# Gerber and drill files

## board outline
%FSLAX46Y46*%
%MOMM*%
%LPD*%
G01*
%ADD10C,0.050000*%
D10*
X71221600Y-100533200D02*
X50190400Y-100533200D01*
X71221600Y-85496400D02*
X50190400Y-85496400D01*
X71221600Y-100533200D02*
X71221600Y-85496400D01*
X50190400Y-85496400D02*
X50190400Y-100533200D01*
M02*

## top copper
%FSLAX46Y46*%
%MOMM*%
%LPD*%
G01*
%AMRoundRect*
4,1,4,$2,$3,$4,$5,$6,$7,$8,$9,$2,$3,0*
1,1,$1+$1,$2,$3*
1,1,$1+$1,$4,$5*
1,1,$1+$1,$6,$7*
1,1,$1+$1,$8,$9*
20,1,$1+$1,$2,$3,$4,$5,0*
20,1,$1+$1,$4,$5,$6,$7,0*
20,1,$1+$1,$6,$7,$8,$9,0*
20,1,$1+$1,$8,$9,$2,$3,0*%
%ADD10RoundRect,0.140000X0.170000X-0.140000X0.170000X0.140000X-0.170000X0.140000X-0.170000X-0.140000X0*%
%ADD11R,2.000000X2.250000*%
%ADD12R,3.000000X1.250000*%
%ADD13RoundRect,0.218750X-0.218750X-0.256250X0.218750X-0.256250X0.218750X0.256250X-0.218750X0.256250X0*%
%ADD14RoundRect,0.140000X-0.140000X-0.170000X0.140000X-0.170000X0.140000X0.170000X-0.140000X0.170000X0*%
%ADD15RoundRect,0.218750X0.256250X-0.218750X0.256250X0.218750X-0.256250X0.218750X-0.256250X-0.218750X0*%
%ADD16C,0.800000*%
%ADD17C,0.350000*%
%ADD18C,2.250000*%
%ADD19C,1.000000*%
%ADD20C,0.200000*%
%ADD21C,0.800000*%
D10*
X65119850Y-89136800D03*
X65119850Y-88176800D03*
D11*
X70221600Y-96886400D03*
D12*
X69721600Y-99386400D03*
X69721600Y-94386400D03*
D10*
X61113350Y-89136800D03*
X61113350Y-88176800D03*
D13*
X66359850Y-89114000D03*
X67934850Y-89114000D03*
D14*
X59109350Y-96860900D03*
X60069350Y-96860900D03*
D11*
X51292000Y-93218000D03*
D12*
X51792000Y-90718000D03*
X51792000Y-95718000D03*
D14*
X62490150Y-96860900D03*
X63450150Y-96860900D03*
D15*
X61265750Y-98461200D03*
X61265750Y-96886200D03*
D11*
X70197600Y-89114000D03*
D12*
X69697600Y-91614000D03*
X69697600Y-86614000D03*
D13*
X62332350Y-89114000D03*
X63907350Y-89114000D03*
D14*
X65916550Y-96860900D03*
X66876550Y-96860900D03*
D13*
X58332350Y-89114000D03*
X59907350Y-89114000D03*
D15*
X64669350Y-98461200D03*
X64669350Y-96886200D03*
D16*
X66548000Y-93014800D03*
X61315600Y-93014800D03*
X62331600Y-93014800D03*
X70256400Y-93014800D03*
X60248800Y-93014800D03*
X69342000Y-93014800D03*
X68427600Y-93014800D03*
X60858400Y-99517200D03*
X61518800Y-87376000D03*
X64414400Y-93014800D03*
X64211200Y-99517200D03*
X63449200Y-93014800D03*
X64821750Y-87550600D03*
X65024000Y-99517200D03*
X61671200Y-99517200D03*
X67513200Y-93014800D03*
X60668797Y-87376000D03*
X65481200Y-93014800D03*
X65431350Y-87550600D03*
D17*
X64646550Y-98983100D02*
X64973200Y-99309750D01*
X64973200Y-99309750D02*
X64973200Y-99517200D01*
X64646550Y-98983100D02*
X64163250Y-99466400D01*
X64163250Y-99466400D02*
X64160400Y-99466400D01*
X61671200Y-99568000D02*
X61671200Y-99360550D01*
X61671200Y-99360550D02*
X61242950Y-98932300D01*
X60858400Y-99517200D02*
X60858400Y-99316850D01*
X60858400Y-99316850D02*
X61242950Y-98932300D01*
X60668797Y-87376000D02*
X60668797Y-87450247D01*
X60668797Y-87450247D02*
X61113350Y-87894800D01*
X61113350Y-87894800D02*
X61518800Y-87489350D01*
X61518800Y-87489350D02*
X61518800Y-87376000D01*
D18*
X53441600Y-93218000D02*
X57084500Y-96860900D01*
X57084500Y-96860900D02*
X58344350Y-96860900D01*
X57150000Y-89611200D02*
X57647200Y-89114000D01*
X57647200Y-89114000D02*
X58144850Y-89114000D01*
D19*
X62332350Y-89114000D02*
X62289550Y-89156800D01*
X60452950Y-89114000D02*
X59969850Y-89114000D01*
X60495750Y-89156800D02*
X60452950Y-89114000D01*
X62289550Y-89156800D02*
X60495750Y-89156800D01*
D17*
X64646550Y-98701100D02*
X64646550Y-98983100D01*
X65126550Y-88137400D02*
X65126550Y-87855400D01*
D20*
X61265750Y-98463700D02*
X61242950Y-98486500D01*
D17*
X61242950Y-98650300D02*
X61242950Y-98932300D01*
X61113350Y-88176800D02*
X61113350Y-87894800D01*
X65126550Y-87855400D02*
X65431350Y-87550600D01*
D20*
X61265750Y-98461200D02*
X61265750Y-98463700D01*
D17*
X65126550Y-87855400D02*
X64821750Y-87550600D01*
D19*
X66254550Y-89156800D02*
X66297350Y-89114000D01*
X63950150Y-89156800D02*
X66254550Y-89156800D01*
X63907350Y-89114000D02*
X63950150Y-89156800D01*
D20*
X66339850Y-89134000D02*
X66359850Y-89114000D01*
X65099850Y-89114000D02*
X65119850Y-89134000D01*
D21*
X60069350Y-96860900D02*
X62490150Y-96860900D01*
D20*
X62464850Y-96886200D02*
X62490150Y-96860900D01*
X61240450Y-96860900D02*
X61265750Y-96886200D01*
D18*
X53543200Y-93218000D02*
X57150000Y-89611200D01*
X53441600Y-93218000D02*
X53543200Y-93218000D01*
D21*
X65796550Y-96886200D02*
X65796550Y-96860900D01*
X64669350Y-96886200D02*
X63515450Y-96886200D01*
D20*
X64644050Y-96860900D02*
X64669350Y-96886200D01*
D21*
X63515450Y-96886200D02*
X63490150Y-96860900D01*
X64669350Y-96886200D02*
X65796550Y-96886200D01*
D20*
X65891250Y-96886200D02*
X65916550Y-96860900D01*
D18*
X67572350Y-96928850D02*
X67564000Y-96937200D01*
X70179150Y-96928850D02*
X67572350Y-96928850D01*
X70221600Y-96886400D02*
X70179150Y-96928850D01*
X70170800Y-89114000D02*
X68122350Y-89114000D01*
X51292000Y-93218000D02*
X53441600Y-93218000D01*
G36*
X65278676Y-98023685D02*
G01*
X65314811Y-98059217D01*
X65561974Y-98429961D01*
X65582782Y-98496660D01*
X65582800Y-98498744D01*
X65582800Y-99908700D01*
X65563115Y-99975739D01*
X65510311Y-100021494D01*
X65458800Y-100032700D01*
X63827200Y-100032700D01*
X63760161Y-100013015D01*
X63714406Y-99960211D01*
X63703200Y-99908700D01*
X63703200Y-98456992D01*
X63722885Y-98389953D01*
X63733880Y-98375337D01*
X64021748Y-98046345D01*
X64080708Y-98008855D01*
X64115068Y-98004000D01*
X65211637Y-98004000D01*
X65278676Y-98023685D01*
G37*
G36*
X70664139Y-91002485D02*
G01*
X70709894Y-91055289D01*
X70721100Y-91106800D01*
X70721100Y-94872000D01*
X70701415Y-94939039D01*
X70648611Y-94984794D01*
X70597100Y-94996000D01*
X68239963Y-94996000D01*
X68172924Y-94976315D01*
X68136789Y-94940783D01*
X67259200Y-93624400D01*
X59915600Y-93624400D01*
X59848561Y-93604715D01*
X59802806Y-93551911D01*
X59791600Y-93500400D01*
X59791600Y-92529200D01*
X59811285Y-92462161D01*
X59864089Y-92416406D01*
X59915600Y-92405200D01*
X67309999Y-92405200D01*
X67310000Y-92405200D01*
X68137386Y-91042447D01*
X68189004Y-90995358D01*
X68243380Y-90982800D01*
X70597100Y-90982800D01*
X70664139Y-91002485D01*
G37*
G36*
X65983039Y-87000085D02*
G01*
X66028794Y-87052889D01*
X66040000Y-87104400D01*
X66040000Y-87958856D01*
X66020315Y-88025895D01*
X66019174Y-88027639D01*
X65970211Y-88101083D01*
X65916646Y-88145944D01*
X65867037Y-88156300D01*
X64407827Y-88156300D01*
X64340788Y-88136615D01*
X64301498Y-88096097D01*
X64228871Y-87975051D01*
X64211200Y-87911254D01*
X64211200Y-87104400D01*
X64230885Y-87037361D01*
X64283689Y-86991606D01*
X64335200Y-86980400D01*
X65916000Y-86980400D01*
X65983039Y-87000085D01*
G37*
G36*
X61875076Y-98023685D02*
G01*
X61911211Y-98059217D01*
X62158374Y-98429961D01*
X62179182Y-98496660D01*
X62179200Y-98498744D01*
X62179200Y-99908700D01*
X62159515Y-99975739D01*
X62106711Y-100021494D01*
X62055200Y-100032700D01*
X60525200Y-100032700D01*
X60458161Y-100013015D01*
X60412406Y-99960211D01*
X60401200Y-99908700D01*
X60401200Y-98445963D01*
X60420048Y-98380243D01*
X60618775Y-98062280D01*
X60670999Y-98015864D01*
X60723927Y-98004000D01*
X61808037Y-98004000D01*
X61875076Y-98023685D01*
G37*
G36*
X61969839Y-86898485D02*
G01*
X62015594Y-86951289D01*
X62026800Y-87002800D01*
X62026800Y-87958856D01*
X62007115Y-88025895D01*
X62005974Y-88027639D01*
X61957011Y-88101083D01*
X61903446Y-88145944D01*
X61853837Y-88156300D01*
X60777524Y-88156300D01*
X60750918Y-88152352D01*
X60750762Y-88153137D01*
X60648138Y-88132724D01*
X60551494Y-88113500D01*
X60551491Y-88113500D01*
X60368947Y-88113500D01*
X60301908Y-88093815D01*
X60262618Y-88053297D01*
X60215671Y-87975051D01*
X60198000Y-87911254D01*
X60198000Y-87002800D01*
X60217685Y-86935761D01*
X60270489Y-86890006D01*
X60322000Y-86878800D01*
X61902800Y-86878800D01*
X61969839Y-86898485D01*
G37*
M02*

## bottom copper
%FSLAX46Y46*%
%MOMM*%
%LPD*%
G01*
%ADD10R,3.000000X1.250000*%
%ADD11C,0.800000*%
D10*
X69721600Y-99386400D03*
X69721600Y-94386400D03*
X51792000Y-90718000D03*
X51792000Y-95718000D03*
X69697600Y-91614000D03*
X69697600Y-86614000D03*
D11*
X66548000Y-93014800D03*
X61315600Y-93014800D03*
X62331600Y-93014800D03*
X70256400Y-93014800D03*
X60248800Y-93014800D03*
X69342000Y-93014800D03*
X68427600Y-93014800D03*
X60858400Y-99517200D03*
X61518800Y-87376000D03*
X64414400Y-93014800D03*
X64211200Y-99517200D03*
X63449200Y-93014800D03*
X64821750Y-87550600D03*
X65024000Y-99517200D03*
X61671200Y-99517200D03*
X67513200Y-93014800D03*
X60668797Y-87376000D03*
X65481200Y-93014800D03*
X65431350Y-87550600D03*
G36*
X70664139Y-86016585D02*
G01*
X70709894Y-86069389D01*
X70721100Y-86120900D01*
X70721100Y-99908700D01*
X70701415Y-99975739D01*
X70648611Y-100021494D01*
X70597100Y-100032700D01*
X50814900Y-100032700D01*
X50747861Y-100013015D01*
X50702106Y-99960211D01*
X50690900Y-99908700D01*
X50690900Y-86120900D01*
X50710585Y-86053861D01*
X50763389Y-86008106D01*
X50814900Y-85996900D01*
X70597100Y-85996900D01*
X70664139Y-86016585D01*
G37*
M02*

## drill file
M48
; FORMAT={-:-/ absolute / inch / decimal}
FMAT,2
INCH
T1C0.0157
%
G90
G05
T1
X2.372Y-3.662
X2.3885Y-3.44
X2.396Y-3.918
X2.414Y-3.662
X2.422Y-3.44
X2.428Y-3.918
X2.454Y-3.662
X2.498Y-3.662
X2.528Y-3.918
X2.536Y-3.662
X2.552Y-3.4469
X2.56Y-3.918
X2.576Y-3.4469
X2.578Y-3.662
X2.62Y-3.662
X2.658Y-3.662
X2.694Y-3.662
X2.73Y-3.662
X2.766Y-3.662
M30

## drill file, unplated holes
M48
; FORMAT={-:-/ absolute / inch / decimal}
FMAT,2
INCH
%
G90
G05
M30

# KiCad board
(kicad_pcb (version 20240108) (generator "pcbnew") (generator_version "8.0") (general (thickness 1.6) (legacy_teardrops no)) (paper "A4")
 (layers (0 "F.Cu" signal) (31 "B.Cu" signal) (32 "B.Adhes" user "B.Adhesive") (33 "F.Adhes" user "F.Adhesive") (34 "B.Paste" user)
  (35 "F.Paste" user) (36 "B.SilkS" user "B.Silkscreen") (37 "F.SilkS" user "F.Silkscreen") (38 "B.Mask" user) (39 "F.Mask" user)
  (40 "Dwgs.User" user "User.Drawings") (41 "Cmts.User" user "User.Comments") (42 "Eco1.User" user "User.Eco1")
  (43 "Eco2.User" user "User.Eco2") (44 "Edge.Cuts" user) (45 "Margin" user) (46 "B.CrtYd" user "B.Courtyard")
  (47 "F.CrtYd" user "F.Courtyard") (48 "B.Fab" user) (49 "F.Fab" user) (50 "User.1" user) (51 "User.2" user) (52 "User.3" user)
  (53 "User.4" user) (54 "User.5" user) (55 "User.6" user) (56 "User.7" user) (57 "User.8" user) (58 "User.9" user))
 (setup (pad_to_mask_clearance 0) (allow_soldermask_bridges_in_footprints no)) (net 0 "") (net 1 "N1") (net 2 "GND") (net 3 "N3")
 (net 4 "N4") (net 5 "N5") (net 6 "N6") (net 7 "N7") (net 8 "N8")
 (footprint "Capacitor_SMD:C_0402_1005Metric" (layer "F.Cu") (at 65.11985 88.6568 90)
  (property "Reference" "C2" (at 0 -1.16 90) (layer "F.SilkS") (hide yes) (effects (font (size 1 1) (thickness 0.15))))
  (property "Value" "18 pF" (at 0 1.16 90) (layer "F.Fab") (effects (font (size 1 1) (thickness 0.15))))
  (pad "1" smd roundrect (at -0.48 0 90) (size 0.56 0.62) (layers "F.Cu" "F.Paste" "F.Mask") (roundrect_rratio 0.25) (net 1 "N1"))
  (pad "2" smd roundrect (at 0.48 0 90) (size 0.56 0.62) (layers "F.Cu" "F.Paste" "F.Mask") (roundrect_rratio 0.25) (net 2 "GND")))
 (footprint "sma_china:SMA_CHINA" (layer "F.Cu") (at 71.2216 96.8864 90)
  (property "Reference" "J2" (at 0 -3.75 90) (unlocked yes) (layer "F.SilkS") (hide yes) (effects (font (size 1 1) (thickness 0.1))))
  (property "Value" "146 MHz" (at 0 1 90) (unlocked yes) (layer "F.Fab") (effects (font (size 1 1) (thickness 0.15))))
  (pad "1" smd rect (at 0 -1 90) (size 2.25 2) (layers "F.Cu" "F.Paste" "F.Mask") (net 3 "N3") (thermal_bridge_angle 45))
  (pad "2" smd rect (at -2.5 -1.5 90) (size 1.25 3) (layers "F.Cu" "F.Paste" "F.Mask") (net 2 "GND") (thermal_bridge_angle 45))
  (pad "2" smd rect (at -2.5 -1.5 90) (size 1.25 3) (layers "B.Cu" "F.Paste" "F.Mask") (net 2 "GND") (thermal_bridge_angle 45))
  (pad "2" smd rect (at 2.5 -1.5 90) (size 1.25 3) (layers "F.Cu" "F.Paste" "F.Mask") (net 2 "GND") (thermal_bridge_angle 45))
  (pad "2" smd rect (at 2.5 -1.5 90) (size 1.25 3) (layers "B.Cu" "F.Paste" "F.Mask") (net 2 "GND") (thermal_bridge_angle 45)))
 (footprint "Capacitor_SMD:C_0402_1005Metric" (layer "F.Cu") (at 61.11335 88.6568 90)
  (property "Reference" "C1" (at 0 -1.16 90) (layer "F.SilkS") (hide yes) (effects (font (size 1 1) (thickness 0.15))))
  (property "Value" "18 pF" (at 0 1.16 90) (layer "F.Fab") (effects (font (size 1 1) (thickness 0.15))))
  (pad "1" smd roundrect (at -0.48 0 90) (size 0.56 0.62) (layers "F.Cu" "F.Paste" "F.Mask") (roundrect_rratio 0.25) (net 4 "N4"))
  (pad "2" smd roundrect (at 0.48 0 90) (size 0.56 0.62) (layers "F.Cu" "F.Paste" "F.Mask") (roundrect_rratio 0.25) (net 2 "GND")))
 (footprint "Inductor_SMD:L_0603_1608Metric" (layer "F.Cu") (at 67.14735 89.114)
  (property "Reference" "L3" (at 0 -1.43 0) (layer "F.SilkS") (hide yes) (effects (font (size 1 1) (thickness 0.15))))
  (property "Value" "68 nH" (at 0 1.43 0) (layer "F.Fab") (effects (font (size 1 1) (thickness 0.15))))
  (pad "1" smd roundrect (at -0.7875 0) (size 0.875 0.95) (layers "F.Cu" "F.Paste" "F.Mask") (roundrect_rratio 0.25) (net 1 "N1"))
  (pad "2" smd roundrect (at 0.7875 0) (size 0.875 0.95) (layers "F.Cu" "F.Paste" "F.Mask") (roundrect_rratio 0.25) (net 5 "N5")))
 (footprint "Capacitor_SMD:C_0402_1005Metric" (layer "F.Cu") (at 59.58935 96.8609)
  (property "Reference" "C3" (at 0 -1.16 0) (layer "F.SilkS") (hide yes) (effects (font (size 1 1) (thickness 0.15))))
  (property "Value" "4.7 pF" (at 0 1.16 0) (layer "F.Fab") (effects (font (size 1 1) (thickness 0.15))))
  (pad "1" smd roundrect (at -0.48 0) (size 0.56 0.62) (layers "F.Cu" "F.Paste" "F.Mask") (roundrect_rratio 0.25) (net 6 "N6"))
  (pad "2" smd roundrect (at 0.48 0) (size 0.56 0.62) (layers "F.Cu" "F.Paste" "F.Mask") (roundrect_rratio 0.25) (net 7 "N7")))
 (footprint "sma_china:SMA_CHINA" (layer "F.Cu") (at 50.292 93.218 -90)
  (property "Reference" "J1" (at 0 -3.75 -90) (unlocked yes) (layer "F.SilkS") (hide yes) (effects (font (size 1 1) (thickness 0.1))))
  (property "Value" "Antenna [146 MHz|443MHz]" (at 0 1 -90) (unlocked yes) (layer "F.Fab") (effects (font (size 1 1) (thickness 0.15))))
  (pad "1" smd rect (at 0 -1 270) (size 2.25 2) (layers "F.Cu" "F.Paste" "F.Mask") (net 6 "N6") (thermal_bridge_angle 45))
  (pad "2" smd rect (at -2.5 -1.5 270) (size 1.25 3) (layers "F.Cu" "F.Paste" "F.Mask") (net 2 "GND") (thermal_bridge_angle 45))
  (pad "2" smd rect (at -2.5 -1.5 270) (size 1.25 3) (layers "B.Cu" "F.Paste" "F.Mask") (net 2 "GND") (thermal_bridge_angle 45))
  (pad "2" smd rect (at 2.5 -1.5 270) (size 1.25 3) (layers "F.Cu" "F.Paste" "F.Mask") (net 2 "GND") (thermal_bridge_angle 45))
  (pad "2" smd rect (at 2.5 -1.5 270) (size 1.25 3) (layers "B.Cu" "F.Paste" "F.Mask") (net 2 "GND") (thermal_bridge_angle 45)))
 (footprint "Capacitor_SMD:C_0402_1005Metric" (layer "F.Cu") (at 62.97015 96.8609)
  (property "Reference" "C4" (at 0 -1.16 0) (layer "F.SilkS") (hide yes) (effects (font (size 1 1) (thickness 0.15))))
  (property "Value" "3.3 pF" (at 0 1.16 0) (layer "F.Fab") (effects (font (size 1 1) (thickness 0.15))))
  (pad "1" smd roundrect (at -0.48 0) (size 0.56 0.62) (layers "F.Cu" "F.Paste" "F.Mask") (roundrect_rratio 0.25) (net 7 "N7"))
  (pad "2" smd roundrect (at 0.48 0) (size 0.56 0.62) (layers "F.Cu" "F.Paste" "F.Mask") (roundrect_rratio 0.25) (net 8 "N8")))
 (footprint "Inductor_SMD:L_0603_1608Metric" (layer "F.Cu") (at 61.26575 97.6737 90)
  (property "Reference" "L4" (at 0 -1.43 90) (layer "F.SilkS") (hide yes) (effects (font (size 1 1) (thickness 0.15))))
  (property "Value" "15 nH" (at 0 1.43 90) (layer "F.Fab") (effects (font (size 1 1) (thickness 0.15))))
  (pad "1" smd roundrect (at -0.7875 0 90) (size 0.875 0.95) (layers "F.Cu" "F.Paste" "F.Mask") (roundrect_rratio 0.25) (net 2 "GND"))
  (pad "2" smd roundrect (at 0.7875 0 90) (size 0.875 0.95) (layers "F.Cu" "F.Paste" "F.Mask") (roundrect_rratio 0.25) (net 7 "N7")))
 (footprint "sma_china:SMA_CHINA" (layer "F.Cu") (at 71.1976 89.114 90)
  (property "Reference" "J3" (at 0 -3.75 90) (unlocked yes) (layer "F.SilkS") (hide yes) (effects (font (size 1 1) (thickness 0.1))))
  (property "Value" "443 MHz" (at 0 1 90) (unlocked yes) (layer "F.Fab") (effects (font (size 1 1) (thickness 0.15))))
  (pad "1" smd rect (at 0 -1 90) (size 2.25 2) (layers "F.Cu" "F.Paste" "F.Mask") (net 5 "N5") (thermal_bridge_angle 45))
  (pad "2" smd rect (at -2.5 -1.5 90) (size 1.25 3) (layers "F.Cu" "F.Paste" "F.Mask") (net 2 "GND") (thermal_bridge_angle 45))
  (pad "2" smd rect (at -2.5 -1.5 90) (size 1.25 3) (layers "B.Cu" "F.Paste" "F.Mask") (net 2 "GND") (thermal_bridge_angle 45))
  (pad "2" smd rect (at 2.5 -1.5 90) (size 1.25 3) (layers "F.Cu" "F.Paste" "F.Mask") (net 2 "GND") (thermal_bridge_angle 45))
  (pad "2" smd rect (at 2.5 -1.5 90) (size 1.25 3) (layers "B.Cu" "F.Paste" "F.Mask") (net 2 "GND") (thermal_bridge_angle 45)))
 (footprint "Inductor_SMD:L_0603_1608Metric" (layer "F.Cu") (at 63.11985 89.114)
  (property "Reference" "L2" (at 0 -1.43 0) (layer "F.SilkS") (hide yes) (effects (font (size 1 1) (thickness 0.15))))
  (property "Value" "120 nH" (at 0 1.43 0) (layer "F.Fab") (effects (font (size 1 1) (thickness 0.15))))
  (pad "1" smd roundrect (at -0.7875 0) (size 0.875 0.95) (layers "F.Cu" "F.Paste" "F.Mask") (roundrect_rratio 0.25) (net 4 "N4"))
  (pad "2" smd roundrect (at 0.7875 0) (size 0.875 0.95) (layers "F.Cu" "F.Paste" "F.Mask") (roundrect_rratio 0.25) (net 1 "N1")))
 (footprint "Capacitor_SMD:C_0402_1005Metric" (layer "F.Cu") (at 66.39655 96.8609)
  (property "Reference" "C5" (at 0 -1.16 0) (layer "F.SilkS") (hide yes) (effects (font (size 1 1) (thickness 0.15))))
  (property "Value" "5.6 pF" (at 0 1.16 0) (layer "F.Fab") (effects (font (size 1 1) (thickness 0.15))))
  (pad "1" smd roundrect (at -0.48 0) (size 0.56 0.62) (layers "F.Cu" "F.Paste" "F.Mask") (roundrect_rratio 0.25) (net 8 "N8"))
  (pad "2" smd roundrect (at 0.48 0) (size 0.56 0.62) (layers "F.Cu" "F.Paste" "F.Mask") (roundrect_rratio 0.25) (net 3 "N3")))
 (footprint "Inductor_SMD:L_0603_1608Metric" (layer "F.Cu") (at 59.11985 89.114)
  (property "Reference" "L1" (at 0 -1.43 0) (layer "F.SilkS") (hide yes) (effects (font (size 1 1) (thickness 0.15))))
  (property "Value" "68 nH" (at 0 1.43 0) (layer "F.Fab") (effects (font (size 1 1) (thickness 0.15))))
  (pad "1" smd roundrect (at -0.7875 0) (size 0.875 0.95) (layers "F.Cu" "F.Paste" "F.Mask") (roundrect_rratio 0.25) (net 6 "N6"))
  (pad "2" smd roundrect (at 0.7875 0) (size 0.875 0.95) (layers "F.Cu" "F.Paste" "F.Mask") (roundrect_rratio 0.25) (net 4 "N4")))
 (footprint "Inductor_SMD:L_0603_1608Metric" (layer "F.Cu") (at 64.66935 97.6737 90)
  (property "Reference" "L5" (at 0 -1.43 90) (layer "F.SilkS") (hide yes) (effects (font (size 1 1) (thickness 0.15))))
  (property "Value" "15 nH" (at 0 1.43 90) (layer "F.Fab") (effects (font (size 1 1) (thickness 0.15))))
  (pad "1" smd roundrect (at -0.7875 0 90) (size 0.875 0.95) (layers "F.Cu" "F.Paste" "F.Mask") (roundrect_rratio 0.25) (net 2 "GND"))
  (pad "2" smd roundrect (at 0.7875 0 90) (size 0.875 0.95) (layers "F.Cu" "F.Paste" "F.Mask") (roundrect_rratio 0.25) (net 8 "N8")))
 (gr_line (start 71.2216 100.5332) (end 50.1904 100.5332) (stroke (width 0.05) (type default)) (layer "Edge.Cuts"))
 (gr_line (start 71.2216 85.4964) (end 50.1904 85.4964) (stroke (width 0.05) (type default)) (layer "Edge.Cuts"))
 (gr_line (start 71.2216 100.5332) (end 71.2216 85.4964) (stroke (width 0.05) (type default)) (layer "Edge.Cuts"))
 (gr_line (start 50.1904 85.4964) (end 50.1904 100.5332) (stroke (width 0.05) (type default)) (layer "Edge.Cuts"))
 (segment (start 62.33235 89.114) (end 62.28955 89.1568) (width 1) (layer "F.Cu") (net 4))
 (segment (start 60.45295 89.114) (end 59.96985 89.114) (width 1) (layer "F.Cu") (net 4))
 (segment (start 60.49575 89.1568) (end 60.45295 89.114) (width 1) (layer "F.Cu") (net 4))
 (segment (start 62.28955 89.1568) (end 60.49575 89.1568) (width 1) (layer "F.Cu") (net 4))
 (segment (start 64.16325 99.4664) (end 64.1604 99.4664) (width 0.35) (layer "F.Cu") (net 2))
 (segment (start 64.64655 98.7011) (end 64.64655 98.9831) (width 0.35) (layer "F.Cu") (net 2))
 (segment (start 64.64655 98.9831) (end 64.9732 99.30975) (width 0.35) (layer "F.Cu") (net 2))
 (segment (start 60.668797 87.450247) (end 61.11335 87.8948) (width 0.35) (layer "F.Cu") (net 2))
 (segment (start 65.12655 88.1374) (end 65.12655 87.8554) (width 0.35) (layer "F.Cu") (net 2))
 (segment (start 61.11335 87.8948) (end 61.5188 87.48935) (width 0.35) (layer "F.Cu") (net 2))
 (segment (start 60.668797 87.376) (end 60.668797 87.450247) (width 0.35) (layer "F.Cu") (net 2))
 (segment (start 61.26575 98.4637) (end 61.24295 98.4865) (width 0.2) (layer "F.Cu") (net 2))
 (segment (start 64.9732 99.30975) (end 64.9732 99.5172) (width 0.35) (layer "F.Cu") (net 2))
 (segment (start 61.24295 98.6503) (end 61.24295 98.9323) (width 0.35) (layer "F.Cu") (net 2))
 (segment (start 61.11335 88.1768) (end 61.11335 87.8948) (width 0.35) (layer "F.Cu") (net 2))
 (segment (start 61.6712 99.568) (end 61.6712 99.36055) (width 0.35) (layer "F.Cu") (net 2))
 (segment (start 64.64655 98.9831) (end 64.16325 99.4664) (width 0.35) (layer "F.Cu") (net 2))
 (segment (start 65.12655 87.8554) (end 65.43135 87.5506) (width 0.35) (layer "F.Cu") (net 2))
 (segment (start 60.8584 99.5172) (end 60.8584 99.31685) (width 0.35) (layer "F.Cu") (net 2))
 (segment (start 61.5188 87.48935) (end 61.5188 87.376) (width 0.35) (layer "F.Cu") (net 2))
 (segment (start 61.26575 98.4612) (end 61.26575 98.4637) (width 0.2) (layer "F.Cu") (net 2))
 (segment (start 65.12655 87.8554) (end 64.82175 87.5506) (width 0.35) (layer "F.Cu") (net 2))
 (segment (start 60.8584 99.31685) (end 61.24295 98.9323) (width 0.35) (layer "F.Cu") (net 2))
 (segment (start 61.6712 99.36055) (end 61.24295 98.9323) (width 0.35) (layer "F.Cu") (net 2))
 (via (at 66.548 93.0148) (size 0.8) (drill 0.4) (layers "F.Cu" "B.Cu") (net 2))
 (via (at 61.3156 93.0148) (size 0.8) (drill 0.4) (layers "F.Cu" "B.Cu") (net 2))
 (via (at 62.3316 93.0148) (size 0.8) (drill 0.4) (layers "F.Cu" "B.Cu") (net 2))
 (via (at 70.2564 93.0148) (size 0.8) (drill 0.4) (layers "F.Cu" "B.Cu") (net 2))
 (via (at 60.2488 93.0148) (size 0.8) (drill 0.4) (layers "F.Cu" "B.Cu") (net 2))
 (via (at 69.342 93.0148) (size 0.8) (drill 0.4) (layers "F.Cu" "B.Cu") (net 2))
 (via (at 68.4276 93.0148) (size 0.8) (drill 0.4) (layers "F.Cu" "B.Cu") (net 2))
 (via (at 60.8584 99.5172) (size 0.8) (drill 0.4) (layers "F.Cu" "B.Cu") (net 2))
 (via (at 61.5188 87.376) (size 0.8) (drill 0.4) (layers "F.Cu" "B.Cu") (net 2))
 (via (at 64.4144 93.0148) (size 0.8) (drill 0.4) (layers "F.Cu" "B.Cu") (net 2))
 (via (at 64.2112 99.5172) (size 0.8) (drill 0.4) (layers "F.Cu" "B.Cu") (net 2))
 (via (at 63.4492 93.0148) (size 0.8) (drill 0.4) (layers "F.Cu" "B.Cu") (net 2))
 (via (at 64.82175 87.5506) (size 0.8) (drill 0.4) (layers "F.Cu" "B.Cu") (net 2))
 (via (at 65.024 99.5172) (size 0.8) (drill 0.4) (layers "F.Cu" "B.Cu") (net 2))
 (via (at 61.6712 99.5172) (size 0.8) (drill 0.4) (layers "F.Cu" "B.Cu") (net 2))
 (via (at 67.5132 93.0148) (size 0.8) (drill 0.4) (layers "F.Cu" "B.Cu") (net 2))
 (via (at 60.668797 87.376) (size 0.8) (drill 0.4) (layers "F.Cu" "B.Cu") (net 2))
 (via (at 65.4812 93.0148) (size 0.8) (drill 0.4) (layers "F.Cu" "B.Cu") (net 2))
 (via (at 65.43135 87.5506) (size 0.8) (drill 0.4) (layers "F.Cu" "B.Cu") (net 2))
 (segment (start 66.25455 89.1568) (end 66.29735 89.114) (width 1) (layer "F.Cu") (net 1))
 (segment (start 63.95015 89.1568) (end 66.25455 89.1568) (width 1) (layer "F.Cu") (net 1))
 (segment (start 63.90735 89.114) (end 63.95015 89.1568) (width 1) (layer "F.Cu") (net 1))
 (segment (start 66.33985 89.134) (end 66.35985 89.114) (width 0.2) (layer "F.Cu") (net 1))
 (segment (start 65.09985 89.114) (end 65.11985 89.134) (width 0.2) (layer "F.Cu") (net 1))
 (segment (start 60.06935 96.8609) (end 62.49015 96.8609) (width 0.8) (layer "F.Cu") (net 7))
 (segment (start 62.46485 96.8862) (end 62.49015 96.8609) (width 0.2) (layer "F.Cu") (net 7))
 (segment (start 61.24045 96.8609) (end 61.26575 96.8862) (width 0.2) (layer "F.Cu") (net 7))
 (segment (start 57.0845 96.8609) (end 58.34435 96.8609) (width 2.25) (layer "F.Cu") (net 6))
 (segment (start 57.6472 89.114) (end 58.14485 89.114) (width 2.25) (layer "F.Cu") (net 6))
 (segment (start 53.5432 93.218) (end 57.15 89.6112) (width 2.25) (layer "F.Cu") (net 6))
 (segment (start 53.4416 93.218) (end 57.0845 96.8609) (width 2.25) (layer "F.Cu") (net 6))
 (segment (start 51.292 93.218) (end 53.4416 93.218) (width 2.25) (layer "F.Cu") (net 6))
 (segment (start 57.15 89.6112) (end 57.6472 89.114) (width 2.25) (layer "F.Cu") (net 6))
 (segment (start 53.4416 93.218) (end 53.5432 93.218) (width 2.25) (layer "F.Cu") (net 6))
 (segment (start 65.79655 96.8862) (end 65.79655 96.8609) (width 0.8) (layer "F.Cu") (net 8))
 (segment (start 64.66935 96.8862) (end 63.51545 96.8862) (width 0.8) (layer "F.Cu") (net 8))
 (segment (start 64.64405 96.8609) (end 64.66935 96.8862) (width 0.2) (layer "F.Cu") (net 8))
 (segment (start 63.51545 96.8862) (end 63.49015 96.8609) (width 0.8) (layer "F.Cu") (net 8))
 (segment (start 64.66935 96.8862) (end 65.79655 96.8862) (width 0.8) (layer "F.Cu") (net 8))
 (segment (start 65.89125 96.8862) (end 65.91655 96.8609) (width 0.2) (layer "F.Cu") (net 8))
 (segment (start 67.57235 96.92885) (end 67.564 96.9372) (width 2.25) (layer "F.Cu") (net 3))
 (segment (start 70.17915 96.92885) (end 67.57235 96.92885) (width 2.25) (layer "F.Cu") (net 3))
 (segment (start 70.2216 96.8864) (end 70.17915 96.92885) (width 2.25) (layer "F.Cu") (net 3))
 (segment (start 70.1708 89.114) (end 68.12235 89.114) (width 2.25) (layer "F.Cu") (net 5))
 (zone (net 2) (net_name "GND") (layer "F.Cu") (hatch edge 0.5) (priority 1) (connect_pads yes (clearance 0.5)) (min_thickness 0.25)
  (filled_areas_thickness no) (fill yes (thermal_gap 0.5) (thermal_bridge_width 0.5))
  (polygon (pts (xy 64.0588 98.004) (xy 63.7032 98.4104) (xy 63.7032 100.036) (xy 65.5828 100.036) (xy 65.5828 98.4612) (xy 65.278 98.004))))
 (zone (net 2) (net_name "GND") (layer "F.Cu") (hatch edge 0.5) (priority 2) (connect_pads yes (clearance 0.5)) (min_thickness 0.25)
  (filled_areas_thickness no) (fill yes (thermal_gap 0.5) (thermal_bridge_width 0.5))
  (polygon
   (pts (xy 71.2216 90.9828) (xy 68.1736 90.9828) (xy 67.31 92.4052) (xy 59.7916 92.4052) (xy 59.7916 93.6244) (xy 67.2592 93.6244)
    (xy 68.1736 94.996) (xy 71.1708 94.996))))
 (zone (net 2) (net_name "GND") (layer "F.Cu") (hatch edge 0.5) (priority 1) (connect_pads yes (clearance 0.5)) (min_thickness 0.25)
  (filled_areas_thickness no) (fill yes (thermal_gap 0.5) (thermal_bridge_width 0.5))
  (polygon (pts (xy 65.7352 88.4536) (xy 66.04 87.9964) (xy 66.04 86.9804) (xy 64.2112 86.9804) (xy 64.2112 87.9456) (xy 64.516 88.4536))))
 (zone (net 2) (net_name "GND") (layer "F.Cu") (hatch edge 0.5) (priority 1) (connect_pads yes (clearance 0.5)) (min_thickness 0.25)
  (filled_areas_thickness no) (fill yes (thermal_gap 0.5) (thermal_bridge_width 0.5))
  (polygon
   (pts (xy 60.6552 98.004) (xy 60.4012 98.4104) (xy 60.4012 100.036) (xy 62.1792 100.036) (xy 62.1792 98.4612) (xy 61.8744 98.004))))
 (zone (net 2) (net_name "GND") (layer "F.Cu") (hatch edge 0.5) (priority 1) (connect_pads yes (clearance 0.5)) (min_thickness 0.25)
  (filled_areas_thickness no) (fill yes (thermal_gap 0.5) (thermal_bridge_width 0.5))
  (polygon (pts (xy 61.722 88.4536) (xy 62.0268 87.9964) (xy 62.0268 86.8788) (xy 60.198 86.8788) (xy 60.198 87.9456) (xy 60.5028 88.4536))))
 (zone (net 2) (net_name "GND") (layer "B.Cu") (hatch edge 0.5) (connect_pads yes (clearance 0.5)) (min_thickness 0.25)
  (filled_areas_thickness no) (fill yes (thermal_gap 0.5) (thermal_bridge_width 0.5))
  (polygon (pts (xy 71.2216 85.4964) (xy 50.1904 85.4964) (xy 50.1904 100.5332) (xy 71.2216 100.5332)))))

